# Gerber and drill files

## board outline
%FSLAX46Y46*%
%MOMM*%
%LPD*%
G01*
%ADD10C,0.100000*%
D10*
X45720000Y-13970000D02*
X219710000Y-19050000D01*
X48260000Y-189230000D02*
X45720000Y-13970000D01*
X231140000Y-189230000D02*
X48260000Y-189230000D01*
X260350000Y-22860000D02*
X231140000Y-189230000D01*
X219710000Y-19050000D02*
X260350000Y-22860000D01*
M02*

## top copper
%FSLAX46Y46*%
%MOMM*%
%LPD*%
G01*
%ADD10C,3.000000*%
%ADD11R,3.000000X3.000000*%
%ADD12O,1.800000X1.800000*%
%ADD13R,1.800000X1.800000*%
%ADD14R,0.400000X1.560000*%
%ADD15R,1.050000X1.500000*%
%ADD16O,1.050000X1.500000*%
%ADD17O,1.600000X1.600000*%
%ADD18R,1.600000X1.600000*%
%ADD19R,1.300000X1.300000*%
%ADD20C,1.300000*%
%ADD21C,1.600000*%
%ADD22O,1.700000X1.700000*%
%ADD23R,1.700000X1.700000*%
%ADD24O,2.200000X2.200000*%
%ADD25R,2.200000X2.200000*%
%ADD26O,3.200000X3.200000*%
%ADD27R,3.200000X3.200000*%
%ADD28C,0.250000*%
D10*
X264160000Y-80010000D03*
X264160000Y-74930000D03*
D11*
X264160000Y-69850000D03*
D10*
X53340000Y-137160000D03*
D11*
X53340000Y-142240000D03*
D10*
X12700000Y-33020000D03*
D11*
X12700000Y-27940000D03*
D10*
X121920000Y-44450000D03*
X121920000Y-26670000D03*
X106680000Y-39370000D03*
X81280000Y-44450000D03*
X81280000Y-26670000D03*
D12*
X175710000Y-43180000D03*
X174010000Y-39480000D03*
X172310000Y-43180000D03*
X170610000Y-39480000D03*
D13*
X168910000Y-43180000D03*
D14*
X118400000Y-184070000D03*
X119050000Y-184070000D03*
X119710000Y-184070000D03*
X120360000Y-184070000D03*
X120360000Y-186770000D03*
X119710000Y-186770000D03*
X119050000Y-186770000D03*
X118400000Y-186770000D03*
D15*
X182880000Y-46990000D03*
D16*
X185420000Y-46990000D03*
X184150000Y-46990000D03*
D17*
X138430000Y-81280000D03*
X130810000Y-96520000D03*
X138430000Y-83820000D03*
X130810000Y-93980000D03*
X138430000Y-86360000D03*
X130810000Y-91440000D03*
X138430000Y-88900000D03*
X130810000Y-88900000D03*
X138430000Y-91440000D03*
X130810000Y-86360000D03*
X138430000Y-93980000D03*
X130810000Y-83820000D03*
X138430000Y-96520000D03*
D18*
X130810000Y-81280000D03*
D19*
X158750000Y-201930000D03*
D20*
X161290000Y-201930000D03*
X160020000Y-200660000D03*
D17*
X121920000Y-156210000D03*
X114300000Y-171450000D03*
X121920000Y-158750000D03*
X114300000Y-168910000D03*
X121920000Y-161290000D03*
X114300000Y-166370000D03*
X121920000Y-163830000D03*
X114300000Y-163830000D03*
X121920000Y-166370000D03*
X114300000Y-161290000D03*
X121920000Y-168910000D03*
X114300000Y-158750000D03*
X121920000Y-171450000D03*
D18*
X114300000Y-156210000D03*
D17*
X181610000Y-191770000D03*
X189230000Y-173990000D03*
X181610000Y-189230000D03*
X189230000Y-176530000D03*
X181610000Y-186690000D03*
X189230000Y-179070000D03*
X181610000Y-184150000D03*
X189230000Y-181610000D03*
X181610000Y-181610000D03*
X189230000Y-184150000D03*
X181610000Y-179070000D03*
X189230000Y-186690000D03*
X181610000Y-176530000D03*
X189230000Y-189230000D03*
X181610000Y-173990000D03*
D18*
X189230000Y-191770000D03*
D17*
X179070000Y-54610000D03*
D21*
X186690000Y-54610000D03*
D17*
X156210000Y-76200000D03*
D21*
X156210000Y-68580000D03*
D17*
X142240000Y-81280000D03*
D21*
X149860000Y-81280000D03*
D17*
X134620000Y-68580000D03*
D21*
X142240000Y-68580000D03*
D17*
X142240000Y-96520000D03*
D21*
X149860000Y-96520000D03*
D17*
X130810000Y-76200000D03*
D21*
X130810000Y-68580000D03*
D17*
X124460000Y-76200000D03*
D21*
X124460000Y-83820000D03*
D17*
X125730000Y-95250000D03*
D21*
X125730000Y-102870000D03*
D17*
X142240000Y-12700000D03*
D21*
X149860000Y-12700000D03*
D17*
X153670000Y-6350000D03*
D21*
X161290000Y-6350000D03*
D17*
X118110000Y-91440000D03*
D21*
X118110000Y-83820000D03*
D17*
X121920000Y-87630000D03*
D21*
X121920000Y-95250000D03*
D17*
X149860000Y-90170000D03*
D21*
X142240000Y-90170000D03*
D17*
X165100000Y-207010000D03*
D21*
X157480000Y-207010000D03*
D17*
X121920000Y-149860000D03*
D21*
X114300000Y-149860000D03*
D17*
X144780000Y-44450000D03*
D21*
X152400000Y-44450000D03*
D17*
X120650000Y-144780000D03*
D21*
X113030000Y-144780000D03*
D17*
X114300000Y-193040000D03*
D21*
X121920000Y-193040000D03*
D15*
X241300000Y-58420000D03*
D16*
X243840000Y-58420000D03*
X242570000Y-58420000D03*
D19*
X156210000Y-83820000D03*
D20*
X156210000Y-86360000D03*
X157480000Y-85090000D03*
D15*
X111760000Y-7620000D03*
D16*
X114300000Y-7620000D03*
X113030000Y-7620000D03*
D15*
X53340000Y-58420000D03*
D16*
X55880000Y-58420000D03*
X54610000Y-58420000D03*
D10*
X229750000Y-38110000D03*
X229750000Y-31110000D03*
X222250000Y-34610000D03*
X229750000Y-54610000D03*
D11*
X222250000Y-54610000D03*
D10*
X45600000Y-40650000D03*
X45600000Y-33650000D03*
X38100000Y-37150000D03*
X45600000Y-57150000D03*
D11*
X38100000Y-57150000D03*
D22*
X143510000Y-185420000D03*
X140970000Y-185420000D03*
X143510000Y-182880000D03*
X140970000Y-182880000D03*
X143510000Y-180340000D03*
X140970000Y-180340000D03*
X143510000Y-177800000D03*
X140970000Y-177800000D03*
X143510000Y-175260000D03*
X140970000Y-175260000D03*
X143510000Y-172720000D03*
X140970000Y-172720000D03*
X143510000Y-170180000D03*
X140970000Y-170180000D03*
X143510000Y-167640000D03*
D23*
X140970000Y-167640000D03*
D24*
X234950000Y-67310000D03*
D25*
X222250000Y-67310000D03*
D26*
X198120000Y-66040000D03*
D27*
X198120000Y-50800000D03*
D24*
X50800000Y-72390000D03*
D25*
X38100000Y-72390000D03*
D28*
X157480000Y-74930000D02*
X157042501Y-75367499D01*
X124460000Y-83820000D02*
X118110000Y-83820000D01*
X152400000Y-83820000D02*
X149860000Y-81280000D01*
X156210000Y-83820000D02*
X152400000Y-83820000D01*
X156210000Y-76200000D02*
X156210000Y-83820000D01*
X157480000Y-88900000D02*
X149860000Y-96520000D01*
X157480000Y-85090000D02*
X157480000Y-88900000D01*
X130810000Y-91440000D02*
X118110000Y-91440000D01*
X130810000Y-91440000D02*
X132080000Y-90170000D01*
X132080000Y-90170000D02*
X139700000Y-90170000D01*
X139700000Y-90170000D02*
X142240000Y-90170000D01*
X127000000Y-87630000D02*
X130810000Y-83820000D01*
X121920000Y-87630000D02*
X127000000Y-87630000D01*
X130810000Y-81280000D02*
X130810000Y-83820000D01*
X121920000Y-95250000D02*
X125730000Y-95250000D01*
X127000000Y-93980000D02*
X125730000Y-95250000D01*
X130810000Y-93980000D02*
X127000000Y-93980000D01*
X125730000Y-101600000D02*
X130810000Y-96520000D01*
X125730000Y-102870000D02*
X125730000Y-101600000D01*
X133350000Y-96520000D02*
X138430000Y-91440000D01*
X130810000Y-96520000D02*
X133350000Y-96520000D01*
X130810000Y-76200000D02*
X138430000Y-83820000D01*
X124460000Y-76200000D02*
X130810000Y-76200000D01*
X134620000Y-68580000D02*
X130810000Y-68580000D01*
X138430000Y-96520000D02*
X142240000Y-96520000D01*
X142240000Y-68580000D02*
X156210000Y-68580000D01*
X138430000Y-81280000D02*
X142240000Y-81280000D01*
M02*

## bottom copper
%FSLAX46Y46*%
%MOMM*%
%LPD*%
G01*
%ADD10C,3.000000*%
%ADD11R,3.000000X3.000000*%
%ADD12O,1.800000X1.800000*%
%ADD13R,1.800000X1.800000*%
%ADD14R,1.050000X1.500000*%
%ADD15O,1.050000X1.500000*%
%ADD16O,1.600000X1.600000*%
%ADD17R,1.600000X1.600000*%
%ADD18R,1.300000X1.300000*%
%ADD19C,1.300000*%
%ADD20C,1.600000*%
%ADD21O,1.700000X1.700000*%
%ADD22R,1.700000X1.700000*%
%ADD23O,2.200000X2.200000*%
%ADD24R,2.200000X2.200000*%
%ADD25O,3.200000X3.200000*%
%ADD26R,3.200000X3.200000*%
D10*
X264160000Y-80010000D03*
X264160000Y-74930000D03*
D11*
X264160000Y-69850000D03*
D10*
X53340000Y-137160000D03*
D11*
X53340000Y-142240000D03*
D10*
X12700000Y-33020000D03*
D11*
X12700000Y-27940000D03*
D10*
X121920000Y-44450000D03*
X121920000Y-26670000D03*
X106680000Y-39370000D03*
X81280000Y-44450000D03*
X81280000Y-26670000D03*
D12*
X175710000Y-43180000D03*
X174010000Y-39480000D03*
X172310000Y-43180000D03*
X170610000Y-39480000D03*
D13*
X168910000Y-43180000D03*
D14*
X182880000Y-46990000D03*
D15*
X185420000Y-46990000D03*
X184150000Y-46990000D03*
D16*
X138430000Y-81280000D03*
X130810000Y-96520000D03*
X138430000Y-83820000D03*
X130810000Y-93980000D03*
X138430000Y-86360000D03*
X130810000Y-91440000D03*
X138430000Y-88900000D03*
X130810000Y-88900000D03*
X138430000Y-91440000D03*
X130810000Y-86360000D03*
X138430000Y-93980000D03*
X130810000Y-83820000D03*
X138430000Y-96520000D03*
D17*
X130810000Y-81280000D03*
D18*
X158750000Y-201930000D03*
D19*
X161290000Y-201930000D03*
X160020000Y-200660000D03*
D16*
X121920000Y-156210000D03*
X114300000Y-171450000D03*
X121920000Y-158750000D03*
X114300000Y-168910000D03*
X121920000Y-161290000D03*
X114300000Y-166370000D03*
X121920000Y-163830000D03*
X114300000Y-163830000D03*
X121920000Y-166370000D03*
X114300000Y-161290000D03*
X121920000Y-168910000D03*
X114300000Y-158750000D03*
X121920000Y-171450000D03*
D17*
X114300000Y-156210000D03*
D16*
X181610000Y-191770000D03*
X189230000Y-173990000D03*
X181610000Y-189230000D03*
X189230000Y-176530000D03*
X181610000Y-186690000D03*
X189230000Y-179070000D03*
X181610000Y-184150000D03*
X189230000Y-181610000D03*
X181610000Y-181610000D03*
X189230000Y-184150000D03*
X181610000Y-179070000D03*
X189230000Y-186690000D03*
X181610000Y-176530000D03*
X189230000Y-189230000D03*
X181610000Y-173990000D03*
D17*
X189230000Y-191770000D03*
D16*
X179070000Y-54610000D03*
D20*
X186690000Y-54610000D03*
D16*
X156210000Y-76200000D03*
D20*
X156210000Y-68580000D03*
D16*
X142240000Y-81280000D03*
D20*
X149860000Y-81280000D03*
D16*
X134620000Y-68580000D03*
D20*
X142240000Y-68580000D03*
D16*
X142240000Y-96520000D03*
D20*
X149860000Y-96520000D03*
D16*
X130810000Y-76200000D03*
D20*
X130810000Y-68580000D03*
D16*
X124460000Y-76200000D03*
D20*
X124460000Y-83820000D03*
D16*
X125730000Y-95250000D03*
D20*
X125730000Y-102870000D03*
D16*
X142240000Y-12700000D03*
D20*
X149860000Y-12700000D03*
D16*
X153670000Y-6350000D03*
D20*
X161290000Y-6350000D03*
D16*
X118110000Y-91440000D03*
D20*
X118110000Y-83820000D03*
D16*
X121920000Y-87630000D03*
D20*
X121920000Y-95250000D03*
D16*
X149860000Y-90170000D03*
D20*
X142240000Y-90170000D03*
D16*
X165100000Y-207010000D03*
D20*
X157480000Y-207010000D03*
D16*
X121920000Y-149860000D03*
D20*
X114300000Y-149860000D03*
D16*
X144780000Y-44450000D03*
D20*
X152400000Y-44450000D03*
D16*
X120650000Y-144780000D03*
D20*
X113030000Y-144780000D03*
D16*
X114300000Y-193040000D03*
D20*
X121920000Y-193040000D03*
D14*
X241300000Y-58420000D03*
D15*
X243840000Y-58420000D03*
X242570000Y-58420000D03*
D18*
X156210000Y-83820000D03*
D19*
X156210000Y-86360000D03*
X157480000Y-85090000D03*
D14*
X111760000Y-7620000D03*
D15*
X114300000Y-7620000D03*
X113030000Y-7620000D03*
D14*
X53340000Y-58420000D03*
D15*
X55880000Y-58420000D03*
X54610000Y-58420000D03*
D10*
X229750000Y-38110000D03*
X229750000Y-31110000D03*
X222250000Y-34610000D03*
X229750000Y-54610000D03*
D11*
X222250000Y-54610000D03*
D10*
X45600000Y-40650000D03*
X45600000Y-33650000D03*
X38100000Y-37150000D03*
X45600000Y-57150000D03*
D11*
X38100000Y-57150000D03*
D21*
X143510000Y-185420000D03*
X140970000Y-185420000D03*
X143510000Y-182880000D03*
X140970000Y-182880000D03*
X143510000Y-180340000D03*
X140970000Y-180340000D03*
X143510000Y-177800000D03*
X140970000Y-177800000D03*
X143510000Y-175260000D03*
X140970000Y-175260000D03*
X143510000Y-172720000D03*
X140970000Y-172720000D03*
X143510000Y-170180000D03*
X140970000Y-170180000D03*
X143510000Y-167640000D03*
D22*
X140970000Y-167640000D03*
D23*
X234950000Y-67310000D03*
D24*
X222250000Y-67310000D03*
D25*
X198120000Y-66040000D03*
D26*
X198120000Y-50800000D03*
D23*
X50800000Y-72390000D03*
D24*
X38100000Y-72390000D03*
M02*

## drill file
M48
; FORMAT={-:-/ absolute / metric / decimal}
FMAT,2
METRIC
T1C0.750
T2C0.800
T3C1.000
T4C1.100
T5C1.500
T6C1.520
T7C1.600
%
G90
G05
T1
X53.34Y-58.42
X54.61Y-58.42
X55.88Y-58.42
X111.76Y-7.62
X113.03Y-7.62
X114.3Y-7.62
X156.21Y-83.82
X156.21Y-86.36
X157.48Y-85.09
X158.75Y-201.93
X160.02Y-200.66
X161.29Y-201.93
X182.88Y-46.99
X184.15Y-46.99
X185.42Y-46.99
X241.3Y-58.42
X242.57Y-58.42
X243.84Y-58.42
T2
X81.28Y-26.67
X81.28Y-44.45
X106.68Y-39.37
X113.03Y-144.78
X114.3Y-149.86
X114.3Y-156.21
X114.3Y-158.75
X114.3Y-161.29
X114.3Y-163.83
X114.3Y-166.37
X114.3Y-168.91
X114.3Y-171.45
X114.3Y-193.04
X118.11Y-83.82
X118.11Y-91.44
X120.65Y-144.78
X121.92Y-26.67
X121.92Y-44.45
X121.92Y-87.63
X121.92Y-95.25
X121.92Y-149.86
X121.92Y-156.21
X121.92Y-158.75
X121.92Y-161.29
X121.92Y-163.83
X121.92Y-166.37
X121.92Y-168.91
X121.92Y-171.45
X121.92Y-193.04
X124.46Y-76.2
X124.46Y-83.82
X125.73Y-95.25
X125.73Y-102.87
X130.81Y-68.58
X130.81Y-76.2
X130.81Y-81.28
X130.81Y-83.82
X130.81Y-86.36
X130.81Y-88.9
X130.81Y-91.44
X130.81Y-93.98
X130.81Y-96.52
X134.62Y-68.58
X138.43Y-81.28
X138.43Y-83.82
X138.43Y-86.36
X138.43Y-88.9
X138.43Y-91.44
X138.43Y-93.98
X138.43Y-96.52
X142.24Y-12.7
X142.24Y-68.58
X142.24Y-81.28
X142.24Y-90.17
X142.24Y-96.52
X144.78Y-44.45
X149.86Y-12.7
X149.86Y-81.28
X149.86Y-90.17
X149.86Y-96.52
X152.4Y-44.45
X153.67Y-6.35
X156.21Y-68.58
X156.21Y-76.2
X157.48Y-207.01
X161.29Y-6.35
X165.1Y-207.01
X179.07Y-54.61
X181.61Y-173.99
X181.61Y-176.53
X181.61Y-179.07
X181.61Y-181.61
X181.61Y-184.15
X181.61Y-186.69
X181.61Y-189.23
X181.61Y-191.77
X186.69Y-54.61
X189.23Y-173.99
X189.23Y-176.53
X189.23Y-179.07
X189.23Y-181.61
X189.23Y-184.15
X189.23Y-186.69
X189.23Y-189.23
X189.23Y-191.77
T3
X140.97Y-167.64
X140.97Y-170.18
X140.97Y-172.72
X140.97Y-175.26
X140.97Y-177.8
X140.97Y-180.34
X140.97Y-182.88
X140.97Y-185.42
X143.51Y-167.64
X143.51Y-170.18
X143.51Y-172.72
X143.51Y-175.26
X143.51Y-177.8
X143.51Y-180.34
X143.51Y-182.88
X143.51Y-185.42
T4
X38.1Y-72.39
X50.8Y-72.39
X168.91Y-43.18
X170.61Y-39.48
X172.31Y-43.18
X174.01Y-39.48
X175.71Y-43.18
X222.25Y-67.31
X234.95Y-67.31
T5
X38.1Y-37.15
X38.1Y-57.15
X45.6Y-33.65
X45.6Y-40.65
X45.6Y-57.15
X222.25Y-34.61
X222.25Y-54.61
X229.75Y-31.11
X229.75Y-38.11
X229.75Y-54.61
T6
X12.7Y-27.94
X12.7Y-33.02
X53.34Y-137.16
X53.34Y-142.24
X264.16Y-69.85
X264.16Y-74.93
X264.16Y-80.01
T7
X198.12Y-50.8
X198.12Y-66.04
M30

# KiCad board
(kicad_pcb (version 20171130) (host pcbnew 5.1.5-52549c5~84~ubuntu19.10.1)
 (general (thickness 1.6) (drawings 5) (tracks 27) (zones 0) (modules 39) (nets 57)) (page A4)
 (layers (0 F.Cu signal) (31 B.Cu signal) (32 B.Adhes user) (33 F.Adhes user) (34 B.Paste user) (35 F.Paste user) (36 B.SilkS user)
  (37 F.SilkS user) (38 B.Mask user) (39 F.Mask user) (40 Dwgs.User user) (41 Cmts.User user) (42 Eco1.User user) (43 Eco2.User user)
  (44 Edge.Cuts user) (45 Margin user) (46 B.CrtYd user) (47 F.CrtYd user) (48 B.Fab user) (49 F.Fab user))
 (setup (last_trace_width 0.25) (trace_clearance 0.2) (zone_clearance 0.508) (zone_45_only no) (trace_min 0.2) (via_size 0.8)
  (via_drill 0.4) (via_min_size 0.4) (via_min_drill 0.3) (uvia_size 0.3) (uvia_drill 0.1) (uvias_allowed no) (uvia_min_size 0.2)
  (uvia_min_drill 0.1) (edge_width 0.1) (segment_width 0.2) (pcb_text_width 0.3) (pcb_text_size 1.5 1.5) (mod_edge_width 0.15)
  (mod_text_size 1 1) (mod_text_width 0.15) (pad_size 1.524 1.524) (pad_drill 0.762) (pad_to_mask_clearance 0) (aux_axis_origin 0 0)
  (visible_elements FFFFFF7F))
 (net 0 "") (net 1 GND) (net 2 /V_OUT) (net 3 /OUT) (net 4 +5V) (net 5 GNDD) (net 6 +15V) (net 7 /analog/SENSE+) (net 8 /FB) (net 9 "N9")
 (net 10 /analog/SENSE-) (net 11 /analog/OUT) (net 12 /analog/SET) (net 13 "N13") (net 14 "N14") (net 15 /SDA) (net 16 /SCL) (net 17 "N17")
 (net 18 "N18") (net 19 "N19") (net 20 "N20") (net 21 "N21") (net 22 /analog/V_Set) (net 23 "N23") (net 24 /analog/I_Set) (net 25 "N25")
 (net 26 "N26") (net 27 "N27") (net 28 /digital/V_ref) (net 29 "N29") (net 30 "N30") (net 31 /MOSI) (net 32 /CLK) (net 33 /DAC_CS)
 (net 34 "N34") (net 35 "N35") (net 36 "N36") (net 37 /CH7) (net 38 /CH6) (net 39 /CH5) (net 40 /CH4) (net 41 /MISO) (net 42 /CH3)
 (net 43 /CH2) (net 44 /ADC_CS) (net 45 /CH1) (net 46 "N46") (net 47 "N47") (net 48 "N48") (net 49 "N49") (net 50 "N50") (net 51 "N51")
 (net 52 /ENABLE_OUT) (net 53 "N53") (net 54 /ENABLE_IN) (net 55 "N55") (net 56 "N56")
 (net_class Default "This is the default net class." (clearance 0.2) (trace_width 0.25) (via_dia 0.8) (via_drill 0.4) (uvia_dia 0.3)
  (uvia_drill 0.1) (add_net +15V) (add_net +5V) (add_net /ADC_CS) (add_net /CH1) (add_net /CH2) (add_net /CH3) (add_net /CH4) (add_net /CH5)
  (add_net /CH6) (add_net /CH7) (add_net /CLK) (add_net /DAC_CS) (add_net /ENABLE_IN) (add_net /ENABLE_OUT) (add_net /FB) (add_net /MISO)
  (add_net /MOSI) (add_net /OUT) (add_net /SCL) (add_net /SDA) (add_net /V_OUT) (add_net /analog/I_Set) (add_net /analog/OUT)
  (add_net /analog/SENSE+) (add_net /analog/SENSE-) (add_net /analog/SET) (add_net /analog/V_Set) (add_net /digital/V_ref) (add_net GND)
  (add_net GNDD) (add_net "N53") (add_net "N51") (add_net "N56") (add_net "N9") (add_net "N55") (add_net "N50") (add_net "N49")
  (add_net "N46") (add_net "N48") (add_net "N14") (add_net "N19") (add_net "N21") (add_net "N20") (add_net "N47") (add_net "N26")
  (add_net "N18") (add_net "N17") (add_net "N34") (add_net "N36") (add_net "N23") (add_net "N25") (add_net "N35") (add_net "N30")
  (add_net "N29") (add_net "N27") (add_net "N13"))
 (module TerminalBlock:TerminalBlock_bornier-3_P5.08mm (layer F.Cu) (at 264.16 69.85 270)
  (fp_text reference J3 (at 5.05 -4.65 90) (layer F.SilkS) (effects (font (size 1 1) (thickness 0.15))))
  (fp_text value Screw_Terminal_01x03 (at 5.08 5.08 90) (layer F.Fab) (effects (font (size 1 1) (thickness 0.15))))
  (pad 3 thru_hole circle (at 10.16 0 270) (size 3 3) (drill 1.52) (layers *.Cu *.Mask) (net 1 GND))
  (pad 2 thru_hole circle (at 5.08 0 270) (size 3 3) (drill 1.52) (layers *.Cu *.Mask) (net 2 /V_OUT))
  (pad 1 thru_hole rect (at 0 0 270) (size 3 3) (drill 1.52) (layers *.Cu *.Mask) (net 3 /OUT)))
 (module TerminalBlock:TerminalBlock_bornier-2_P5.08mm (layer F.Cu) (at 53.34 142.24 90)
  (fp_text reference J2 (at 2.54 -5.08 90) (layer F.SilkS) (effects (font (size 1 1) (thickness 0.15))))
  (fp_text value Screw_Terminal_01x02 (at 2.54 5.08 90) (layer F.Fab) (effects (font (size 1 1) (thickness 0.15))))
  (pad 2 thru_hole circle (at 5.08 0 90) (size 3 3) (drill 1.52) (layers *.Cu *.Mask) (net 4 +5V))
  (pad 1 thru_hole rect (at 0 0 90) (size 3 3) (drill 1.52) (layers *.Cu *.Mask) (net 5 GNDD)))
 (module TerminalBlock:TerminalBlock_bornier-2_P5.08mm (layer F.Cu) (at 12.7 27.94 270)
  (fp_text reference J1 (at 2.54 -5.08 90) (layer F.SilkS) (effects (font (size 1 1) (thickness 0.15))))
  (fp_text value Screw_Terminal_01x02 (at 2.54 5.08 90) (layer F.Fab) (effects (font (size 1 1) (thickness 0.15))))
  (pad 2 thru_hole circle (at 5.08 0 270) (size 3 3) (drill 1.52) (layers *.Cu *.Mask) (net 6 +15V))
  (pad 1 thru_hole rect (at 0 0 270) (size 3 3) (drill 1.52) (layers *.Cu *.Mask) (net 1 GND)))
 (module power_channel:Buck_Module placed (layer F.Cu) (at 101.6 35.56)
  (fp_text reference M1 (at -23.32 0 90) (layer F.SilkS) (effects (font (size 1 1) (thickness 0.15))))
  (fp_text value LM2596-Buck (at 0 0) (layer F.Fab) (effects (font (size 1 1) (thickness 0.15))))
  (pad 3 thru_hole circle (at 20.32 8.89) (size 3 3) (drill 0.8) (layers *.Cu *.Mask) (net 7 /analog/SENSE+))
  (pad 4 thru_hole circle (at 20.32 -8.89) (size 3 3) (drill 0.8) (layers *.Cu *.Mask) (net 1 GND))
  (pad 2 thru_hole circle (at 5.08 3.81) (size 3 3) (drill 0.8) (layers *.Cu *.Mask) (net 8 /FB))
  (pad 1 thru_hole circle (at -20.32 8.89) (size 3 3) (drill 0.8) (layers *.Cu *.Mask) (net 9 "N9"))
  (pad 5 thru_hole circle (at -20.32 -8.89) (size 3 3) (drill 0.8) (layers *.Cu *.Mask) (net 1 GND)))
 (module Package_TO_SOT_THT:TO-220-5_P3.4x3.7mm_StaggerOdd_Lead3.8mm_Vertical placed (layer F.Cu) (at 168.91 43.18)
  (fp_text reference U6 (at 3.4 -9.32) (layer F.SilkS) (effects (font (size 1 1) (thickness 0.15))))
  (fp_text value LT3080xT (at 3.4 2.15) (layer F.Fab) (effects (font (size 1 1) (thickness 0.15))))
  (pad 5 thru_hole oval (at 6.8 0) (size 1.8 1.8) (drill 1.1) (layers *.Cu *.Mask) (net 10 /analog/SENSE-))
  (pad 4 thru_hole oval (at 5.1 -3.7) (size 1.8 1.8) (drill 1.1) (layers *.Cu *.Mask) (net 6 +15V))
  (pad 3 thru_hole oval (at 3.4 0) (size 1.8 1.8) (drill 1.1) (layers *.Cu *.Mask) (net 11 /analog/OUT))
  (pad 2 thru_hole oval (at 1.7 -3.7) (size 1.8 1.8) (drill 1.1) (layers *.Cu *.Mask) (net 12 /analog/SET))
  (pad 1 thru_hole rect (at 0 0) (size 1.8 1.8) (drill 1.1) (layers *.Cu *.Mask) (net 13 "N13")))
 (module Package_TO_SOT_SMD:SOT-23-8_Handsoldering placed (layer F.Cu) (at 119.38 185.42 90)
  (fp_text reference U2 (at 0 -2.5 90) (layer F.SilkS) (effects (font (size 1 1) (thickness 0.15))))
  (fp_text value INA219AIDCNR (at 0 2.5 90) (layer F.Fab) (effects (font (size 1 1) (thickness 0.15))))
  (pad 8 smd rect (at 1.35 -0.98 90) (size 1.56 0.4) (layers F.Cu F.Paste F.Mask) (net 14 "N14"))
  (pad 7 smd rect (at 1.35 -0.33 90) (size 1.56 0.4) (layers F.Cu F.Paste F.Mask) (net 14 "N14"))
  (pad 6 smd rect (at 1.35 0.33 90) (size 1.56 0.4) (layers F.Cu F.Paste F.Mask) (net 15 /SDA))
  (pad 5 smd rect (at 1.35 0.98 90) (size 1.56 0.4) (layers F.Cu F.Paste F.Mask) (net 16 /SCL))
  (pad 4 smd rect (at -1.35 0.98 90) (size 1.56 0.4) (layers F.Cu F.Paste F.Mask) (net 4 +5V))
  (pad 3 smd rect (at -1.35 0.33 90) (size 1.56 0.4) (layers F.Cu F.Paste F.Mask) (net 5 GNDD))
  (pad 2 smd rect (at -1.35 -0.33 90) (size 1.56 0.4) (layers F.Cu F.Paste F.Mask) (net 10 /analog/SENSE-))
  (pad 1 smd rect (at -1.35 -0.98 90) (size 1.56 0.4) (layers F.Cu F.Paste F.Mask) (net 7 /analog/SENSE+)))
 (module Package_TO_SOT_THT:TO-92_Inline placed (layer F.Cu) (at 182.88 46.99)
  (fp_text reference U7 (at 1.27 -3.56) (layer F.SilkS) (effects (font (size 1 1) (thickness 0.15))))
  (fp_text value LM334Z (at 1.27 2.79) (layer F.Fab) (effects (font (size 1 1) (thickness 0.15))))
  (pad 1 thru_hole rect (at 0 0) (size 1.05 1.5) (drill 0.75) (layers *.Cu *.Mask) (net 11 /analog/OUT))
  (pad 3 thru_hole oval (at 2.54 0) (size 1.05 1.5) (drill 0.75) (layers *.Cu *.Mask) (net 1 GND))
  (pad 2 thru_hole oval (at 1.27 0) (size 1.05 1.5) (drill 0.75) (layers *.Cu *.Mask) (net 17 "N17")))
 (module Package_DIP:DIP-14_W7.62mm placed (layer F.Cu) (at 130.81 81.28)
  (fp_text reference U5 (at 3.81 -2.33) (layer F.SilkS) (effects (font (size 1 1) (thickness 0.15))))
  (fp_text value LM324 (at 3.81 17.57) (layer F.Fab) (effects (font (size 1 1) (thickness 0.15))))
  (pad 14 thru_hole oval (at 7.62 0) (size 1.6 1.6) (drill 0.8) (layers *.Cu *.Mask) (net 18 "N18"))
  (pad 7 thru_hole oval (at 0 15.24) (size 1.6 1.6) (drill 0.8) (layers *.Cu *.Mask) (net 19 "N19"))
  (pad 13 thru_hole oval (at 7.62 2.54) (size 1.6 1.6) (drill 0.8) (layers *.Cu *.Mask) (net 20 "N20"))
  (pad 6 thru_hole oval (at 0 12.7) (size 1.6 1.6) (drill 0.8) (layers *.Cu *.Mask) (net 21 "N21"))
  (pad 12 thru_hole oval (at 7.62 5.08) (size 1.6 1.6) (drill 0.8) (layers *.Cu *.Mask) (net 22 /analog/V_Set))
  (pad 5 thru_hole oval (at 0 10.16) (size 1.6 1.6) (drill 0.8) (layers *.Cu *.Mask) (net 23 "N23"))
  (pad 11 thru_hole oval (at 7.62 7.62) (size 1.6 1.6) (drill 0.8) (layers *.Cu *.Mask) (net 1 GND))
  (pad 4 thru_hole oval (at 0 7.62) (size 1.6 1.6) (drill 0.8) (layers *.Cu *.Mask) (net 6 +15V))
  (pad 10 thru_hole oval (at 7.62 10.16) (size 1.6 1.6) (drill 0.8) (layers *.Cu *.Mask) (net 19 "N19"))
  (pad 3 thru_hole oval (at 0 5.08) (size 1.6 1.6) (drill 0.8) (layers *.Cu *.Mask) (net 10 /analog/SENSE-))
  (pad 9 thru_hole oval (at 7.62 12.7) (size 1.6 1.6) (drill 0.8) (layers *.Cu *.Mask) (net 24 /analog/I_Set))
  (pad 2 thru_hole oval (at 0 2.54) (size 1.6 1.6) (drill 0.8) (layers *.Cu *.Mask) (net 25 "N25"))
  (pad 8 thru_hole oval (at 7.62 15.24) (size 1.6 1.6) (drill 0.8) (layers *.Cu *.Mask) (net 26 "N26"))
  (pad 1 thru_hole rect (at 0 0) (size 1.6 1.6) (drill 0.8) (layers *.Cu *.Mask) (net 25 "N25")))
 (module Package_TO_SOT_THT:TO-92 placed (layer F.Cu) (at 158.75 201.93)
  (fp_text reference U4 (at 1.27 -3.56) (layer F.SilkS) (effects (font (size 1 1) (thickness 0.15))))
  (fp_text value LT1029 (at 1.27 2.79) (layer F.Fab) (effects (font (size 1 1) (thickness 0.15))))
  (pad 1 thru_hole rect (at 0 0 90) (size 1.3 1.3) (drill 0.75) (layers *.Cu *.Mask) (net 5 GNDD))
  (pad 3 thru_hole circle (at 2.54 0 90) (size 1.3 1.3) (drill 0.75) (layers *.Cu *.Mask) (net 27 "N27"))
  (pad 2 thru_hole circle (at 1.27 -1.27 90) (size 1.3 1.3) (drill 0.75) (layers *.Cu *.Mask) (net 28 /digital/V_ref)))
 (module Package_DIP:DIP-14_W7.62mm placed (layer F.Cu) (at 114.3 156.21)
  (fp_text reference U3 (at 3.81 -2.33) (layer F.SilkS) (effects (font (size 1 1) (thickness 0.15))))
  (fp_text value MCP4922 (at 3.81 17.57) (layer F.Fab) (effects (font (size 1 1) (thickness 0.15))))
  (pad 14 thru_hole oval (at 7.62 0) (size 1.6 1.6) (drill 0.8) (layers *.Cu *.Mask) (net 22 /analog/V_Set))
  (pad 7 thru_hole oval (at 0 15.24) (size 1.6 1.6) (drill 0.8) (layers *.Cu *.Mask) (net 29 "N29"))
  (pad 13 thru_hole oval (at 7.62 2.54) (size 1.6 1.6) (drill 0.8) (layers *.Cu *.Mask) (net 28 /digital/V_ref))
  (pad 6 thru_hole oval (at 0 12.7) (size 1.6 1.6) (drill 0.8) (layers *.Cu *.Mask) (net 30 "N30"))
  (pad 12 thru_hole oval (at 7.62 5.08) (size 1.6 1.6) (drill 0.8) (layers *.Cu *.Mask) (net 5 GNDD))
  (pad 5 thru_hole oval (at 0 10.16) (size 1.6 1.6) (drill 0.8) (layers *.Cu *.Mask) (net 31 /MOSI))
  (pad 11 thru_hole oval (at 7.62 7.62) (size 1.6 1.6) (drill 0.8) (layers *.Cu *.Mask) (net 28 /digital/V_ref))
  (pad 4 thru_hole oval (at 0 7.62) (size 1.6 1.6) (drill 0.8) (layers *.Cu *.Mask) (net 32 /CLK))
  (pad 10 thru_hole oval (at 7.62 10.16) (size 1.6 1.6) (drill 0.8) (layers *.Cu *.Mask) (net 24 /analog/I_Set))
  (pad 3 thru_hole oval (at 0 5.08) (size 1.6 1.6) (drill 0.8) (layers *.Cu *.Mask) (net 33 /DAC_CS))
  (pad 9 thru_hole oval (at 7.62 12.7) (size 1.6 1.6) (drill 0.8) (layers *.Cu *.Mask) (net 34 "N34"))
  (pad 2 thru_hole oval (at 0 2.54) (size 1.6 1.6) (drill 0.8) (layers *.Cu *.Mask) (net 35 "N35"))
  (pad 8 thru_hole oval (at 7.62 15.24) (size 1.6 1.6) (drill 0.8) (layers *.Cu *.Mask) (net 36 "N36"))
  (pad 1 thru_hole rect (at 0 0) (size 1.6 1.6) (drill 0.8) (layers *.Cu *.Mask) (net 4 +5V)))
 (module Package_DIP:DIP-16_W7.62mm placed (layer F.Cu) (at 189.23 191.77 180)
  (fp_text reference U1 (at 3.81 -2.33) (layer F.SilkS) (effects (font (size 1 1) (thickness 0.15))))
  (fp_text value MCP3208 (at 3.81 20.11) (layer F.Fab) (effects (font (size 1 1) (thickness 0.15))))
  (pad 16 thru_hole oval (at 7.62 0 180) (size 1.6 1.6) (drill 0.8) (layers *.Cu *.Mask) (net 4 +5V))
  (pad 8 thru_hole oval (at 0 17.78 180) (size 1.6 1.6) (drill 0.8) (layers *.Cu *.Mask) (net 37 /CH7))
  (pad 15 thru_hole oval (at 7.62 2.54 180) (size 1.6 1.6) (drill 0.8) (layers *.Cu *.Mask) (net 28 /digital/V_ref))
  (pad 7 thru_hole oval (at 0 15.24 180) (size 1.6 1.6) (drill 0.8) (layers *.Cu *.Mask) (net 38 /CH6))
  (pad 14 thru_hole oval (at 7.62 5.08 180) (size 1.6 1.6) (drill 0.8) (layers *.Cu *.Mask) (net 1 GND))
  (pad 6 thru_hole oval (at 0 12.7 180) (size 1.6 1.6) (drill 0.8) (layers *.Cu *.Mask) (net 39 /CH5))
  (pad 13 thru_hole oval (at 7.62 7.62 180) (size 1.6 1.6) (drill 0.8) (layers *.Cu *.Mask) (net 32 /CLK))
  (pad 5 thru_hole oval (at 0 10.16 180) (size 1.6 1.6) (drill 0.8) (layers *.Cu *.Mask) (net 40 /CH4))
  (pad 12 thru_hole oval (at 7.62 10.16 180) (size 1.6 1.6) (drill 0.8) (layers *.Cu *.Mask) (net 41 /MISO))
  (pad 4 thru_hole oval (at 0 7.62 180) (size 1.6 1.6) (drill 0.8) (layers *.Cu *.Mask) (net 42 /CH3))
  (pad 11 thru_hole oval (at 7.62 12.7 180) (size 1.6 1.6) (drill 0.8) (layers *.Cu *.Mask) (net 31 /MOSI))
  (pad 3 thru_hole oval (at 0 5.08 180) (size 1.6 1.6) (drill 0.8) (layers *.Cu *.Mask) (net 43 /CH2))
  (pad 10 thru_hole oval (at 7.62 15.24 180) (size 1.6 1.6) (drill 0.8) (layers *.Cu *.Mask) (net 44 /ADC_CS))
  (pad 2 thru_hole oval (at 0 2.54 180) (size 1.6 1.6) (drill 0.8) (layers *.Cu *.Mask) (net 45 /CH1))
  (pad 9 thru_hole oval (at 7.62 17.78 180) (size 1.6 1.6) (drill 0.8) (layers *.Cu *.Mask) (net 5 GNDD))
  (pad 1 thru_hole rect (at 0 0 180) (size 1.6 1.6) (drill 0.8) (layers *.Cu *.Mask) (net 2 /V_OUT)))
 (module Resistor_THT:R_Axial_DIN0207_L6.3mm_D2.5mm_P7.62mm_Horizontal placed (layer F.Cu) (at 186.69 54.61 180)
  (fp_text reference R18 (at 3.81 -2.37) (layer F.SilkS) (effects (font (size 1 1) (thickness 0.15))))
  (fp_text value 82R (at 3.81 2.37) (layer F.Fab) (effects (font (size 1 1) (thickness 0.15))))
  (pad 2 thru_hole oval (at 7.62 0 180) (size 1.6 1.6) (drill 0.8) (layers *.Cu *.Mask) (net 1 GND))
  (pad 1 thru_hole circle (at 0 0 180) (size 1.6 1.6) (drill 0.8) (layers *.Cu *.Mask) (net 17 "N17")))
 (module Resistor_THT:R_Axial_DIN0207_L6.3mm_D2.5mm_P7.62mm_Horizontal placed (layer F.Cu) (at 156.21 68.58 270)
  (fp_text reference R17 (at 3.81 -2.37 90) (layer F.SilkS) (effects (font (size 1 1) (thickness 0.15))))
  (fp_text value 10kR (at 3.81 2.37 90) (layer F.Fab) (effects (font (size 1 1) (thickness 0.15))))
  (pad 2 thru_hole oval (at 7.62 0 270) (size 1.6 1.6) (drill 0.8) (layers *.Cu *.Mask) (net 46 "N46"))
  (pad 1 thru_hole circle (at 0 0 270) (size 1.6 1.6) (drill 0.8) (layers *.Cu *.Mask) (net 12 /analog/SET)))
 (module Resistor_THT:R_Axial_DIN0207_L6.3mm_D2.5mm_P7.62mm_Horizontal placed (layer F.Cu) (at 149.86 81.28 180)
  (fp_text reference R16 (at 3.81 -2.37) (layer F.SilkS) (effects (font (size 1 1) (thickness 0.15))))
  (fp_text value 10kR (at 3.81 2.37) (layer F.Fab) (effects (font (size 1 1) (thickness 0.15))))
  (pad 2 thru_hole oval (at 7.62 0 180) (size 1.6 1.6) (drill 0.8) (layers *.Cu *.Mask) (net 18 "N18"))
  (pad 1 thru_hole circle (at 0 0 180) (size 1.6 1.6) (drill 0.8) (layers *.Cu *.Mask) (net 46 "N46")))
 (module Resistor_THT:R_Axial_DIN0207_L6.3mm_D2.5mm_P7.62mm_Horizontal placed (layer F.Cu) (at 142.24 68.58 180)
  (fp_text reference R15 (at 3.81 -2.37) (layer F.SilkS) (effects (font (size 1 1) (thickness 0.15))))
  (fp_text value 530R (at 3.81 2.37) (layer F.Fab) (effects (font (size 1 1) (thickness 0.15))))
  (pad 2 thru_hole oval (at 7.62 0 180) (size 1.6 1.6) (drill 0.8) (layers *.Cu *.Mask) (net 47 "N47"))
  (pad 1 thru_hole circle (at 0 0 180) (size 1.6 1.6) (drill 0.8) (layers *.Cu *.Mask) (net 12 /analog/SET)))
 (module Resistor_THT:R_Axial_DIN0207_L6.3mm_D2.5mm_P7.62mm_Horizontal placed (layer F.Cu) (at 149.86 96.52 180)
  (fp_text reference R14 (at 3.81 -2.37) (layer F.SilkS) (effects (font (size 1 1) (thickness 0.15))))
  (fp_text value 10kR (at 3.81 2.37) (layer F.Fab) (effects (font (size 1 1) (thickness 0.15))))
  (pad 2 thru_hole oval (at 7.62 0 180) (size 1.6 1.6) (drill 0.8) (layers *.Cu *.Mask) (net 26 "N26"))
  (pad 1 thru_hole circle (at 0 0 180) (size 1.6 1.6) (drill 0.8) (layers *.Cu *.Mask) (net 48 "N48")))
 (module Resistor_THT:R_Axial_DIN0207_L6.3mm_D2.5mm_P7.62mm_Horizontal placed (layer F.Cu) (at 130.81 68.58 270)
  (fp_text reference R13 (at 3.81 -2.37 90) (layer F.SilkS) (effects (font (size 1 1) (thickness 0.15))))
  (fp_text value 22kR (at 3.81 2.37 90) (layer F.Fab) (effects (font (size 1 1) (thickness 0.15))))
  (pad 2 thru_hole oval (at 7.62 0 270) (size 1.6 1.6) (drill 0.8) (layers *.Cu *.Mask) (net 20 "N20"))
  (pad 1 thru_hole circle (at 0 0 270) (size 1.6 1.6) (drill 0.8) (layers *.Cu *.Mask) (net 47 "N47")))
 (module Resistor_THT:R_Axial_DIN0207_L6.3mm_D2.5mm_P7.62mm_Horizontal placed (layer F.Cu) (at 124.46 83.82 90)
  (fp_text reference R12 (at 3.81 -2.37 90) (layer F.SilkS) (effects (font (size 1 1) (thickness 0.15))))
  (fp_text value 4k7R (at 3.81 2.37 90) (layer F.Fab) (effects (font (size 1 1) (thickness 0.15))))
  (pad 2 thru_hole oval (at 7.62 0 90) (size 1.6 1.6) (drill 0.8) (layers *.Cu *.Mask) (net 20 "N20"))
  (pad 1 thru_hole circle (at 0 0 90) (size 1.6 1.6) (drill 0.8) (layers *.Cu *.Mask) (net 1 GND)))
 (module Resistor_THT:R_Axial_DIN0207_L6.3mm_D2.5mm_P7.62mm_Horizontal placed (layer F.Cu) (at 125.73 102.87 90)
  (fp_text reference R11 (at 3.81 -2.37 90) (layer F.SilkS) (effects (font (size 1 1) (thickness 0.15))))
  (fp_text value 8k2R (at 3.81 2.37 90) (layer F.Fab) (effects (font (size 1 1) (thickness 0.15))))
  (pad 2 thru_hole oval (at 7.62 0 90) (size 1.6 1.6) (drill 0.8) (layers *.Cu *.Mask) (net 21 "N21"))
  (pad 1 thru_hole circle (at 0 0 90) (size 1.6 1.6) (drill 0.8) (layers *.Cu *.Mask) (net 19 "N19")))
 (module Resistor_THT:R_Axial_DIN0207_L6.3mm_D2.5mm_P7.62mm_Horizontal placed (layer F.Cu) (at 149.86 12.7 180)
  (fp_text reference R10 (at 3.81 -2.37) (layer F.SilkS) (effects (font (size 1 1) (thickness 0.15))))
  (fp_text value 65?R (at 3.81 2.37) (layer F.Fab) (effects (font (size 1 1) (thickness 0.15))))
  (pad 2 thru_hole oval (at 7.62 0 180) (size 1.6 1.6) (drill 0.8) (layers *.Cu *.Mask) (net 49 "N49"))
  (pad 1 thru_hole circle (at 0 0 180) (size 1.6 1.6) (drill 0.8) (layers *.Cu *.Mask) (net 10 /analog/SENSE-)))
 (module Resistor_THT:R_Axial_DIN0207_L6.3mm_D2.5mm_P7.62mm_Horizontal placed (layer F.Cu) (at 161.29 6.35 180)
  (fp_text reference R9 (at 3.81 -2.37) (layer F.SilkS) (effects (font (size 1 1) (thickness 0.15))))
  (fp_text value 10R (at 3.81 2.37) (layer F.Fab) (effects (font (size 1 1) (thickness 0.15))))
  (pad 2 thru_hole oval (at 7.62 0 180) (size 1.6 1.6) (drill 0.8) (layers *.Cu *.Mask) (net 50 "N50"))
  (pad 1 thru_hole circle (at 0 0 180) (size 1.6 1.6) (drill 0.8) (layers *.Cu *.Mask) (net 11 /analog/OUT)))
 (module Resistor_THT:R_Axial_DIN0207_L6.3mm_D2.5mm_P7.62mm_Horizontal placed (layer F.Cu) (at 118.11 83.82 270)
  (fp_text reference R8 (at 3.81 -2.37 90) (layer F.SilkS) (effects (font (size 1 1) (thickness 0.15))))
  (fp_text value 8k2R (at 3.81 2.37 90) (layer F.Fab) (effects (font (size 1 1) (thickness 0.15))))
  (pad 2 thru_hole oval (at 7.62 0 270) (size 1.6 1.6) (drill 0.8) (layers *.Cu *.Mask) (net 23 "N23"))
  (pad 1 thru_hole circle (at 0 0 270) (size 1.6 1.6) (drill 0.8) (layers *.Cu *.Mask) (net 1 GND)))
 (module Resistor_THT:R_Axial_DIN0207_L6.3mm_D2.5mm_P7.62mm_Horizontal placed (layer F.Cu) (at 121.92 95.25 90)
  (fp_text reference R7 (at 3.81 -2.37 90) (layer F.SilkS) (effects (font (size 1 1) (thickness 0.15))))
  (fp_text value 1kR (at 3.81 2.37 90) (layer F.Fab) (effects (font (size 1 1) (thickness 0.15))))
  (pad 2 thru_hole oval (at 7.62 0 90) (size 1.6 1.6) (drill 0.8) (layers *.Cu *.Mask) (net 25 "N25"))
  (pad 1 thru_hole circle (at 0 0 90) (size 1.6 1.6) (drill 0.8) (layers *.Cu *.Mask) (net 21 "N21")))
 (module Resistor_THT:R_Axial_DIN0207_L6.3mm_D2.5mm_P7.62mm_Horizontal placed (layer F.Cu) (at 142.24 90.17)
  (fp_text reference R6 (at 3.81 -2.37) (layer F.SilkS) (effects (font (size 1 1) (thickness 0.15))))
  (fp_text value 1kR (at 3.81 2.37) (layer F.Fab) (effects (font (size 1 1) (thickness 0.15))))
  (pad 2 thru_hole oval (at 7.62 0) (size 1.6 1.6) (drill 0.8) (layers *.Cu *.Mask) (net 7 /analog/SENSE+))
  (pad 1 thru_hole circle (at 0 0) (size 1.6 1.6) (drill 0.8) (layers *.Cu *.Mask) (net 23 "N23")))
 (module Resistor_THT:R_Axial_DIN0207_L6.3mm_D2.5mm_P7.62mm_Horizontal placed (layer F.Cu) (at 157.48 207.01)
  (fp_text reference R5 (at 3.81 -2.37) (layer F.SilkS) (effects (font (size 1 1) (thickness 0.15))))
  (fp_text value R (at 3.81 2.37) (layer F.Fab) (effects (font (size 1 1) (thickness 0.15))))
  (pad 2 thru_hole oval (at 7.62 0) (size 1.6 1.6) (drill 0.8) (layers *.Cu *.Mask) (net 4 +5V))
  (pad 1 thru_hole circle (at 0 0) (size 1.6 1.6) (drill 0.8) (layers *.Cu *.Mask) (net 28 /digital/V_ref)))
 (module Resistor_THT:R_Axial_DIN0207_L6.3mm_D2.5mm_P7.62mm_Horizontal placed (layer F.Cu) (at 114.3 149.86)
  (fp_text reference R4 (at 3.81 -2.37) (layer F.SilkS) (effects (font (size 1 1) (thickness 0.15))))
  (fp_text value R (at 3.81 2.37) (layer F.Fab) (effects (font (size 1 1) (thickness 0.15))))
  (pad 2 thru_hole oval (at 7.62 0) (size 1.6 1.6) (drill 0.8) (layers *.Cu *.Mask) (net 5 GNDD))
  (pad 1 thru_hole circle (at 0 0) (size 1.6 1.6) (drill 0.8) (layers *.Cu *.Mask) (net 36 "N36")))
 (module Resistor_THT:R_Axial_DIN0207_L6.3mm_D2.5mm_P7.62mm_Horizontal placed (layer F.Cu) (at 152.4 44.45 180)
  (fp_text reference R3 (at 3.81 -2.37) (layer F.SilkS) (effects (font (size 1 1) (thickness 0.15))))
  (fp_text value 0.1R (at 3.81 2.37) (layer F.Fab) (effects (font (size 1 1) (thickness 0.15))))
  (pad 2 thru_hole oval (at 7.62 0 180) (size 1.6 1.6) (drill 0.8) (layers *.Cu *.Mask) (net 7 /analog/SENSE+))
  (pad 1 thru_hole circle (at 0 0 180) (size 1.6 1.6) (drill 0.8) (layers *.Cu *.Mask) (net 10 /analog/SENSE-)))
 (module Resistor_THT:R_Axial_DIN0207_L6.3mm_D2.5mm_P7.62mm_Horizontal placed (layer F.Cu) (at 113.03 144.78)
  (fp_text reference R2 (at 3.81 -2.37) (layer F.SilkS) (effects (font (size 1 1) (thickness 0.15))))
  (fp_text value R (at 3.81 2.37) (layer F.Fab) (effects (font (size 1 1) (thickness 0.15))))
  (pad 2 thru_hole oval (at 7.62 0) (size 1.6 1.6) (drill 0.8) (layers *.Cu *.Mask) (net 4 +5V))
  (pad 1 thru_hole circle (at 0 0) (size 1.6 1.6) (drill 0.8) (layers *.Cu *.Mask) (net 34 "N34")))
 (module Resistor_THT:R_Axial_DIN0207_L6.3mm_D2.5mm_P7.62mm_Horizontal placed (layer F.Cu) (at 121.92 193.04 180)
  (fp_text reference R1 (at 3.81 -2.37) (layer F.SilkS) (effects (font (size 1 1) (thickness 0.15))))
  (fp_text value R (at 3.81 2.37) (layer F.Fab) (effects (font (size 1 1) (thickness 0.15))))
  (pad 2 thru_hole oval (at 7.62 0 180) (size 1.6 1.6) (drill 0.8) (layers *.Cu *.Mask) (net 5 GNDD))
  (pad 1 thru_hole circle (at 0 0 180) (size 1.6 1.6) (drill 0.8) (layers *.Cu *.Mask) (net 14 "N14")))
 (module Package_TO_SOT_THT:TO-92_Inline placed (layer F.Cu) (at 241.3 58.42)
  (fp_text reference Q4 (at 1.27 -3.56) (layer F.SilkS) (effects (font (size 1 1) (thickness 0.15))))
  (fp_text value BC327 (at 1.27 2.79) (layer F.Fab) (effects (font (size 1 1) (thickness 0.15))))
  (pad 1 thru_hole rect (at 0 0) (size 1.05 1.5) (drill 0.75) (layers *.Cu *.Mask) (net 1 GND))
  (pad 3 thru_hole oval (at 2.54 0) (size 1.05 1.5) (drill 0.75) (layers *.Cu *.Mask) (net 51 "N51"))
  (pad 2 thru_hole oval (at 1.27 0) (size 1.05 1.5) (drill 0.75) (layers *.Cu *.Mask) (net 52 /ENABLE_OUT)))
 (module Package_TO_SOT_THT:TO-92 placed (layer F.Cu) (at 156.21 83.82 270)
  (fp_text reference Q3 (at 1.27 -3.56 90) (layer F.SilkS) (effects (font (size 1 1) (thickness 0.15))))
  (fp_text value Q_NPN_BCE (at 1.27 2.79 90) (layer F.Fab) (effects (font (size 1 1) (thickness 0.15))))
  (pad 1 thru_hole rect (at 0 0) (size 1.3 1.3) (drill 0.75) (layers *.Cu *.Mask) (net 46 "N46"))
  (pad 3 thru_hole circle (at 2.54 0) (size 1.3 1.3) (drill 0.75) (layers *.Cu *.Mask) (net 1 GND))
  (pad 2 thru_hole circle (at 1.27 -1.27) (size 1.3 1.3) (drill 0.75) (layers *.Cu *.Mask) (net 48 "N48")))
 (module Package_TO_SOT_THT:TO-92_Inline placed (layer F.Cu) (at 111.76 7.62)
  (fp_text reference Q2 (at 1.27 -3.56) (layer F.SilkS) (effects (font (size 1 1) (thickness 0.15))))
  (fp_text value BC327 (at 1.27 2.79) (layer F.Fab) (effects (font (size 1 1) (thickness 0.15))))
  (pad 1 thru_hole rect (at 0 0) (size 1.05 1.5) (drill 0.75) (layers *.Cu *.Mask) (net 8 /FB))
  (pad 3 thru_hole oval (at 2.54 0) (size 1.05 1.5) (drill 0.75) (layers *.Cu *.Mask) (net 49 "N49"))
  (pad 2 thru_hole oval (at 1.27 0) (size 1.05 1.5) (drill 0.75) (layers *.Cu *.Mask) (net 50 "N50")))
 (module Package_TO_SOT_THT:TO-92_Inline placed (layer F.Cu) (at 53.34 58.42)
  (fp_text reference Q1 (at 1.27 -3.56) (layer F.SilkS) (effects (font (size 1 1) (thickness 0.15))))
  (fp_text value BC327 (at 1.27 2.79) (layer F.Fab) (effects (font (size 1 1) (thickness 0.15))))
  (pad 1 thru_hole rect (at 0 0) (size 1.05 1.5) (drill 0.75) (layers *.Cu *.Mask) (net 1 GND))
  (pad 3 thru_hole oval (at 2.54 0) (size 1.05 1.5) (drill 0.75) (layers *.Cu *.Mask) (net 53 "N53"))
  (pad 2 thru_hole oval (at 1.27 0) (size 1.05 1.5) (drill 0.75) (layers *.Cu *.Mask) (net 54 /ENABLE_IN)))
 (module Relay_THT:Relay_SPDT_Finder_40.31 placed (layer F.Cu) (at 222.25 54.61 90)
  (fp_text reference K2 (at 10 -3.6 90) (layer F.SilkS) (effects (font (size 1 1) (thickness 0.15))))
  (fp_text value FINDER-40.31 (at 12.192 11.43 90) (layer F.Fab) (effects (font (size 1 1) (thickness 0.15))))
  (pad 12 thru_hole circle (at 16.5 7.5 90) (size 3 3) (drill 1.5) (layers *.Cu *.Mask) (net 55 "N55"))
  (pad 14 thru_hole circle (at 23.5 7.5 90) (size 3 3) (drill 1.5) (layers *.Cu *.Mask) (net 3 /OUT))
  (pad 11 thru_hole circle (at 20 0 90) (size 3 3) (drill 1.5) (layers *.Cu *.Mask) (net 11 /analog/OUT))
  (pad A2 thru_hole circle (at 0 7.5 90) (size 3 3) (drill 1.5) (layers *.Cu *.Mask) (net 51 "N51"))
  (pad A1 thru_hole rect (at 0 0 90) (size 3 3) (drill 1.5) (layers *.Cu *.Mask) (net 6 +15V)))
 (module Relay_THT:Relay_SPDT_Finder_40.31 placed (layer F.Cu) (at 38.1 57.15 90)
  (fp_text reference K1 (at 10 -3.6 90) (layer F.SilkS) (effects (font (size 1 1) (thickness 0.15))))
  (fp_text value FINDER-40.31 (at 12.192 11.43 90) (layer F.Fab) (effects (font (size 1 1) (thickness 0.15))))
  (pad 12 thru_hole circle (at 16.5 7.5 90) (size 3 3) (drill 1.5) (layers *.Cu *.Mask) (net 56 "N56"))
  (pad 14 thru_hole circle (at 23.5 7.5 90) (size 3 3) (drill 1.5) (layers *.Cu *.Mask) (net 9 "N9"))
  (pad 11 thru_hole circle (at 20 0 90) (size 3 3) (drill 1.5) (layers *.Cu *.Mask) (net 6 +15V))
  (pad A2 thru_hole circle (at 0 7.5 90) (size 3 3) (drill 1.5) (layers *.Cu *.Mask) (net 53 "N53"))
  (pad A1 thru_hole rect (at 0 0 90) (size 3 3) (drill 1.5) (layers *.Cu *.Mask) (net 6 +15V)))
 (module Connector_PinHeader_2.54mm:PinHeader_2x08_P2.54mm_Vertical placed (layer F.Cu) (at 140.97 167.64)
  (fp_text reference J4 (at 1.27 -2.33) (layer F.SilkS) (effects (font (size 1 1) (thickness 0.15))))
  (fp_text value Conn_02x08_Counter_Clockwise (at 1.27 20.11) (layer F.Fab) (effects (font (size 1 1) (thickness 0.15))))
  (pad 16 thru_hole oval (at 2.54 17.78) (size 1.7 1.7) (drill 1) (layers *.Cu *.Mask) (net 52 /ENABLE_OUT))
  (pad 15 thru_hole oval (at 0 17.78) (size 1.7 1.7) (drill 1) (layers *.Cu *.Mask) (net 45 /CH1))
  (pad 14 thru_hole oval (at 2.54 15.24) (size 1.7 1.7) (drill 1) (layers *.Cu *.Mask) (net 43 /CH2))
  (pad 13 thru_hole oval (at 0 15.24) (size 1.7 1.7) (drill 1) (layers *.Cu *.Mask) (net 42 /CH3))
  (pad 12 thru_hole oval (at 2.54 12.7) (size 1.7 1.7) (drill 1) (layers *.Cu *.Mask) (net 40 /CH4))
  (pad 11 thru_hole oval (at 0 12.7) (size 1.7 1.7) (drill 1) (layers *.Cu *.Mask) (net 39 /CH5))
  (pad 10 thru_hole oval (at 2.54 10.16) (size 1.7 1.7) (drill 1) (layers *.Cu *.Mask) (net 38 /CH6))
  (pad 9 thru_hole oval (at 0 10.16) (size 1.7 1.7) (drill 1) (layers *.Cu *.Mask) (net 37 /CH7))
  (pad 8 thru_hole oval (at 2.54 7.62) (size 1.7 1.7) (drill 1) (layers *.Cu *.Mask) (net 15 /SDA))
  (pad 7 thru_hole oval (at 0 7.62) (size 1.7 1.7) (drill 1) (layers *.Cu *.Mask) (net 16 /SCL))
  (pad 6 thru_hole oval (at 2.54 5.08) (size 1.7 1.7) (drill 1) (layers *.Cu *.Mask) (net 32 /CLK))
  (pad 5 thru_hole oval (at 0 5.08) (size 1.7 1.7) (drill 1) (layers *.Cu *.Mask) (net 31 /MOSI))
  (pad 4 thru_hole oval (at 2.54 2.54) (size 1.7 1.7) (drill 1) (layers *.Cu *.Mask) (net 41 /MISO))
  (pad 3 thru_hole oval (at 0 2.54) (size 1.7 1.7) (drill 1) (layers *.Cu *.Mask) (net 33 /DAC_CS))
  (pad 2 thru_hole oval (at 2.54 0) (size 1.7 1.7) (drill 1) (layers *.Cu *.Mask) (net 44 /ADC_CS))
  (pad 1 thru_hole rect (at 0 0) (size 1.7 1.7) (drill 1) (layers *.Cu *.Mask) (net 54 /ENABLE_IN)))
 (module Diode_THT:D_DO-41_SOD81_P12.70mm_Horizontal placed (layer F.Cu) (at 222.25 67.31)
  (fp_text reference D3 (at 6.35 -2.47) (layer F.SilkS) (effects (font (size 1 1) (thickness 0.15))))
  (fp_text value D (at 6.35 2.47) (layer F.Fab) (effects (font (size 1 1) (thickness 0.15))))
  (pad 2 thru_hole oval (at 12.7 0) (size 2.2 2.2) (drill 1.1) (layers *.Cu *.Mask) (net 51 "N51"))
  (pad 1 thru_hole rect (at 0 0) (size 2.2 2.2) (drill 1.1) (layers *.Cu *.Mask) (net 6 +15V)))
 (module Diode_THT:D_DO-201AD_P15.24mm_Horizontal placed (layer F.Cu) (at 198.12 50.8 270)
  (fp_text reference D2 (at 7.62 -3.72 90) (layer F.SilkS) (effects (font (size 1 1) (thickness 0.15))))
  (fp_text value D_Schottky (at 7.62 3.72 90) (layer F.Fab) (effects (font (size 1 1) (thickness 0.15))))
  (pad 2 thru_hole oval (at 15.24 0 270) (size 3.2 3.2) (drill 1.6) (layers *.Cu *.Mask) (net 1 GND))
  (pad 1 thru_hole rect (at 0 0 270) (size 3.2 3.2) (drill 1.6) (layers *.Cu *.Mask) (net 11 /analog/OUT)))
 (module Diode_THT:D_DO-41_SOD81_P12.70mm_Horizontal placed (layer F.Cu) (at 38.1 72.39)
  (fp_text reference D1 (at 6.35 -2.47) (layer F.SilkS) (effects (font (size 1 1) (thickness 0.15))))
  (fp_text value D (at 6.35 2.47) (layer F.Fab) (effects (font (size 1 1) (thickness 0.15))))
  (pad 2 thru_hole oval (at 12.7 0) (size 2.2 2.2) (drill 1.1) (layers *.Cu *.Mask) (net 53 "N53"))
  (pad 1 thru_hole rect (at 0 0) (size 2.2 2.2) (drill 1.1) (layers *.Cu *.Mask) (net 6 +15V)))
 (gr_line (start 45.72 13.97) (end 219.71 19.05) (layer Edge.Cuts) (width 0.1))
 (gr_line (start 48.26 189.23) (end 45.72 13.97) (layer Edge.Cuts) (width 0.1))
 (gr_line (start 231.14 189.23) (end 48.26 189.23) (layer Edge.Cuts) (width 0.1))
 (gr_line (start 260.35 22.86) (end 231.14 189.23) (layer Edge.Cuts) (width 0.1))
 (gr_line (start 219.71 19.05) (end 260.35 22.86) (layer Edge.Cuts) (width 0.1))
 (segment (start 157.48 74.93) (end 157.042501 75.367499) (width 0.25) (layer F.Cu) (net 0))
 (segment (start 124.46 83.82) (end 118.11 83.82) (width 0.25) (layer F.Cu) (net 1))
 (segment (start 152.4 83.82) (end 149.86 81.28) (width 0.25) (layer F.Cu) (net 46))
 (segment (start 156.21 83.82) (end 152.4 83.82) (width 0.25) (layer F.Cu) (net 46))
 (segment (start 156.21 76.2) (end 156.21 83.82) (width 0.25) (layer F.Cu) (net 46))
 (segment (start 157.48 88.9) (end 149.86 96.52) (width 0.25) (layer F.Cu) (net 48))
 (segment (start 157.48 85.09) (end 157.48 88.9) (width 0.25) (layer F.Cu) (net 48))
 (segment (start 130.81 91.44) (end 118.11 91.44) (width 0.25) (layer F.Cu) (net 23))
 (segment (start 130.81 91.44) (end 132.08 90.17) (width 0.25) (layer F.Cu) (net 23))
 (segment (start 132.08 90.17) (end 139.7 90.17) (width 0.25) (layer F.Cu) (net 23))
 (segment (start 139.7 90.17) (end 142.24 90.17) (width 0.25) (layer F.Cu) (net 23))
 (segment (start 127 87.63) (end 130.81 83.82) (width 0.25) (layer F.Cu) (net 25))
 (segment (start 121.92 87.63) (end 127 87.63) (width 0.25) (layer F.Cu) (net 25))
 (segment (start 130.81 81.28) (end 130.81 83.82) (width 0.25) (layer F.Cu) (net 25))
 (segment (start 121.92 95.25) (end 125.73 95.25) (width 0.25) (layer F.Cu) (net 21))
 (segment (start 127 93.98) (end 125.73 95.25) (width 0.25) (layer F.Cu) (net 21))
 (segment (start 130.81 93.98) (end 127 93.98) (width 0.25) (layer F.Cu) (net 21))
 (segment (start 125.73 101.6) (end 130.81 96.52) (width 0.25) (layer F.Cu) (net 19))
 (segment (start 125.73 102.87) (end 125.73 101.6) (width 0.25) (layer F.Cu) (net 19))
 (segment (start 133.35 96.52) (end 138.43 91.44) (width 0.25) (layer F.Cu) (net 19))
 (segment (start 130.81 96.52) (end 133.35 96.52) (width 0.25) (layer F.Cu) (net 19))
 (segment (start 130.81 76.2) (end 138.43 83.82) (width 0.25) (layer F.Cu) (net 20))
 (segment (start 124.46 76.2) (end 130.81 76.2) (width 0.25) (layer F.Cu) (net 20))
 (segment (start 134.62 68.58) (end 130.81 68.58) (width 0.25) (layer F.Cu) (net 47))
 (segment (start 138.43 96.52) (end 142.24 96.52) (width 0.25) (layer F.Cu) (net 26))
 (segment (start 142.24 68.58) (end 156.21 68.58) (width 0.25) (layer F.Cu) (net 12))
 (segment (start 138.43 81.28) (end 142.24 81.28) (width 0.25) (layer F.Cu) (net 18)))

